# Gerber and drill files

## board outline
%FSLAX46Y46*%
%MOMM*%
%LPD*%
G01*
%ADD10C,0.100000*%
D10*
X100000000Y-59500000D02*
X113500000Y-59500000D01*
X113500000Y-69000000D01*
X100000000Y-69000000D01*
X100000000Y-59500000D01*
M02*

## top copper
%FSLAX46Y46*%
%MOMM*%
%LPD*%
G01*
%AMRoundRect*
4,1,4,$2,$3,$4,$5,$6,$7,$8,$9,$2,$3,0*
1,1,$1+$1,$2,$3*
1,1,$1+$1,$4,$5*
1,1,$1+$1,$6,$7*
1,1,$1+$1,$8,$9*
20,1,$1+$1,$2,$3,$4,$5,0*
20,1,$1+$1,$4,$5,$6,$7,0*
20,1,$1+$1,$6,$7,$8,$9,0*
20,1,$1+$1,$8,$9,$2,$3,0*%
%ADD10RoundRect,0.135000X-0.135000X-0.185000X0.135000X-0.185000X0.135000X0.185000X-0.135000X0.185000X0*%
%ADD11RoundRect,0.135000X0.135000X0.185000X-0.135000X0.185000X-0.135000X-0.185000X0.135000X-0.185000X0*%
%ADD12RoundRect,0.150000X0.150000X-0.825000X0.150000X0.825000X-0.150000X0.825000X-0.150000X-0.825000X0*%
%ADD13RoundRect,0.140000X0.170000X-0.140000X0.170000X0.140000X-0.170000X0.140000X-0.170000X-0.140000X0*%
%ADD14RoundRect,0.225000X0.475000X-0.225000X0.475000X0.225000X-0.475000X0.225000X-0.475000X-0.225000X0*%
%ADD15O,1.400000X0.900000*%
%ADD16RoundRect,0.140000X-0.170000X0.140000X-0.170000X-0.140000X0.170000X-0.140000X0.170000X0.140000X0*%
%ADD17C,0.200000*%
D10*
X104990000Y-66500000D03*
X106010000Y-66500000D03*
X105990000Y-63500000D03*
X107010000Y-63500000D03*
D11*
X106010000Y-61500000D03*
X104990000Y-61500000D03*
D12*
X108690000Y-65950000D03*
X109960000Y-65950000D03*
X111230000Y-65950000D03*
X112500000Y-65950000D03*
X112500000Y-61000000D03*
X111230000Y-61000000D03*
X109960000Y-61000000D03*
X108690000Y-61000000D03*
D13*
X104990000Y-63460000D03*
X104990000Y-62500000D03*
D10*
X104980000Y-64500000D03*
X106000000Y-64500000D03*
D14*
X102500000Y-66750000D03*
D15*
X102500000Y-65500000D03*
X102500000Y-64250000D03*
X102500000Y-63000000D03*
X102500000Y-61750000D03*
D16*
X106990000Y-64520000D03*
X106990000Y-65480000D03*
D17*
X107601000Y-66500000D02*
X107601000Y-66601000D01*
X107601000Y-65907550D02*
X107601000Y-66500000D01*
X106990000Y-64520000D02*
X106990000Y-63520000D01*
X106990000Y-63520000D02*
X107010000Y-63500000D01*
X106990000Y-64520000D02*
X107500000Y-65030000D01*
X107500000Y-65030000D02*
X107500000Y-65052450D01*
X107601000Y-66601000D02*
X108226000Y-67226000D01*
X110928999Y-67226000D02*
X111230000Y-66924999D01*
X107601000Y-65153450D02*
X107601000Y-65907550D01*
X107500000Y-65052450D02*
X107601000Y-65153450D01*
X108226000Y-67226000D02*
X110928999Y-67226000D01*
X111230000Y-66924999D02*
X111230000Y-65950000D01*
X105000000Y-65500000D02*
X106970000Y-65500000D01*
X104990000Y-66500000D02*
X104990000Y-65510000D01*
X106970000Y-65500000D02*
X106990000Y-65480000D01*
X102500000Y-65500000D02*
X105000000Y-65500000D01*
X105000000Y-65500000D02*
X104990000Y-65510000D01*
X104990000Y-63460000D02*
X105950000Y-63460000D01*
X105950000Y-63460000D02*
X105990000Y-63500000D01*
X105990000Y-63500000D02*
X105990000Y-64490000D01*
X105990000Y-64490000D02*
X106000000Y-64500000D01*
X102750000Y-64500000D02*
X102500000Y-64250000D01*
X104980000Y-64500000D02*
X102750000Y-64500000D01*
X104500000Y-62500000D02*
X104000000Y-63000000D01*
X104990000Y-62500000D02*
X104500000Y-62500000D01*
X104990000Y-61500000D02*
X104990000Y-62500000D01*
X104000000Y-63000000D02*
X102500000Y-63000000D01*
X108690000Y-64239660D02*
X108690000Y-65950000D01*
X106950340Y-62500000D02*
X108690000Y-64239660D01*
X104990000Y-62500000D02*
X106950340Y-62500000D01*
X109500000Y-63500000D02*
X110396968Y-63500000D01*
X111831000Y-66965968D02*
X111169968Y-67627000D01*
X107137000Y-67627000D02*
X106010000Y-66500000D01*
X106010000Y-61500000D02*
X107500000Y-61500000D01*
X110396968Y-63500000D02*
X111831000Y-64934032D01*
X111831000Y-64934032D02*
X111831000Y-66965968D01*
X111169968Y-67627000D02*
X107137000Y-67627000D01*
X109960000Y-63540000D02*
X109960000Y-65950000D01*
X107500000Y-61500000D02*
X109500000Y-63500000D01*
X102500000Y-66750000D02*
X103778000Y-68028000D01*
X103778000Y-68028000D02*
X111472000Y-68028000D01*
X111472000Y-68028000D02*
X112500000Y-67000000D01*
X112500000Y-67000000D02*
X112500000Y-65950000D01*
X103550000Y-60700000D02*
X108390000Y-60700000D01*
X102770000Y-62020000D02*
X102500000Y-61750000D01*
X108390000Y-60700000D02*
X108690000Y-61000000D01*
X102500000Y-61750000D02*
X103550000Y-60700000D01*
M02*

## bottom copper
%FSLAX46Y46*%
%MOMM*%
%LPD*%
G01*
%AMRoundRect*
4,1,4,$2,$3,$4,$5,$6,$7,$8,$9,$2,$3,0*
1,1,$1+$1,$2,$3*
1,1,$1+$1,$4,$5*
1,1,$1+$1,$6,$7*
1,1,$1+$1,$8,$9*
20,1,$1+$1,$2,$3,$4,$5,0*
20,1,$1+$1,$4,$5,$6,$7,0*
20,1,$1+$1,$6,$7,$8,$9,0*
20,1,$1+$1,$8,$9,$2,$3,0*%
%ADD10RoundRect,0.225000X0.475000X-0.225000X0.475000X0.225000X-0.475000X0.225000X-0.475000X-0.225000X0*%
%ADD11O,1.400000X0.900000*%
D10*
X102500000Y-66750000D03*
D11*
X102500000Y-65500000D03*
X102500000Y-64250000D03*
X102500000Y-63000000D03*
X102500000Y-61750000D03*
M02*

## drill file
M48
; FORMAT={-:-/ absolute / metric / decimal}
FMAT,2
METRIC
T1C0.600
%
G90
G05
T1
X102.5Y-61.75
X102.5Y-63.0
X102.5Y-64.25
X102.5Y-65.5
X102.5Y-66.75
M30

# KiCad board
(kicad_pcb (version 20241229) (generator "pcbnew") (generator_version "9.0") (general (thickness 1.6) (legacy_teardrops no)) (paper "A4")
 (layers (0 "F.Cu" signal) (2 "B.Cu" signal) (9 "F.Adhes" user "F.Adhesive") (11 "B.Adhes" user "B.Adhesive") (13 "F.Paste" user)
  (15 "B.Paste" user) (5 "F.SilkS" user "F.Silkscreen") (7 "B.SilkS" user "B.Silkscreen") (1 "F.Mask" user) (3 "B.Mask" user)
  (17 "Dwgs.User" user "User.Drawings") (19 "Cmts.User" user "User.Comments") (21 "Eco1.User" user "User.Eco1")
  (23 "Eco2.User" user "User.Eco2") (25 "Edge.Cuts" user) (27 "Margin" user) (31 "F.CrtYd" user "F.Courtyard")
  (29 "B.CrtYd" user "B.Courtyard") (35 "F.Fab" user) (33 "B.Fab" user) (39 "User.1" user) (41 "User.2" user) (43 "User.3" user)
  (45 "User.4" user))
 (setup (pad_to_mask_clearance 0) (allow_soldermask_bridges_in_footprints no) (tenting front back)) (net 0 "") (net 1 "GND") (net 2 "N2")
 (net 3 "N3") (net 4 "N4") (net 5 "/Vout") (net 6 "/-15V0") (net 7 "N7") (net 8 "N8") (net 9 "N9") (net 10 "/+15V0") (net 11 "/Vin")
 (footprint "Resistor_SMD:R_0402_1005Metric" (layer "F.Cu") (at 105.5 66.5)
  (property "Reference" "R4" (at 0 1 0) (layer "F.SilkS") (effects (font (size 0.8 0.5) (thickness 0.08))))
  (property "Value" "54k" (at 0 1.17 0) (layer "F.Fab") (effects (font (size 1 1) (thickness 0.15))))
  (pad "1" smd roundrect (at -0.51 0) (size 0.54 0.64) (layers "F.Cu" "F.Mask" "F.Paste") (roundrect_rratio 0.25) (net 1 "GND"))
  (pad "2" smd roundrect (at 0.51 0) (size 0.54 0.64) (layers "F.Cu" "F.Mask" "F.Paste") (roundrect_rratio 0.25) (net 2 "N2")))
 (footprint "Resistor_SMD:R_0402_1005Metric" (layer "F.Cu") (at 106.5 63.5)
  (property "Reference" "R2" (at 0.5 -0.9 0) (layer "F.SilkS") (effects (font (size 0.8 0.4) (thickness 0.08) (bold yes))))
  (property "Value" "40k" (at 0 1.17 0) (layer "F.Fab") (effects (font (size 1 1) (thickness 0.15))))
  (pad "1" smd roundrect (at -0.51 0) (size 0.54 0.64) (layers "F.Cu" "F.Mask" "F.Paste") (roundrect_rratio 0.25) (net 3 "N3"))
  (pad "2" smd roundrect (at 0.51 0) (size 0.54 0.64) (layers "F.Cu" "F.Mask" "F.Paste") (roundrect_rratio 0.25) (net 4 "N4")))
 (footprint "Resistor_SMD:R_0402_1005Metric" (layer "F.Cu") (at 105.5 61.5 180)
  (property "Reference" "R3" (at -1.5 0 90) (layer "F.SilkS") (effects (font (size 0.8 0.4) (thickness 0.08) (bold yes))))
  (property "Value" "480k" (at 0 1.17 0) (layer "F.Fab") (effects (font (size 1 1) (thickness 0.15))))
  (pad "1" smd roundrect (at -0.51 0 180) (size 0.54 0.64) (layers "F.Cu" "F.Mask" "F.Paste") (roundrect_rratio 0.25) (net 2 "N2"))
  (pad "2" smd roundrect (at 0.51 0 180) (size 0.54 0.64) (layers "F.Cu" "F.Mask" "F.Paste") (roundrect_rratio 0.25) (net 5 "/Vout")))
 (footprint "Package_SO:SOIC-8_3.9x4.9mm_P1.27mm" (layer "F.Cu") (at 110.595 63.475 90)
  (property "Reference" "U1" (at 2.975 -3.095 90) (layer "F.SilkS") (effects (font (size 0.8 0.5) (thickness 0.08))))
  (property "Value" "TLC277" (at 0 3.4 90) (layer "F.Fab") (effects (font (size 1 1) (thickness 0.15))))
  (pad "1" smd roundrect (at -2.475 -1.905 90) (size 1.95 0.6) (layers "F.Cu" "F.Mask" "F.Paste") (roundrect_rratio 0.25) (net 5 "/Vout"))
  (pad "2" smd roundrect (at -2.475 -0.635 90) (size 1.95 0.6) (layers "F.Cu" "F.Mask" "F.Paste") (roundrect_rratio 0.25) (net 2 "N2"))
  (pad "3" smd roundrect (at -2.475 0.635 90) (size 1.95 0.6) (layers "F.Cu" "F.Mask" "F.Paste") (roundrect_rratio 0.25) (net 4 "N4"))
  (pad "4" smd roundrect (at -2.475 1.905 90) (size 1.95 0.6) (layers "F.Cu" "F.Mask" "F.Paste") (roundrect_rratio 0.25) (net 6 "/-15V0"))
  (pad "5" smd roundrect (at 2.475 1.905 90) (size 1.95 0.6) (layers "F.Cu" "F.Mask" "F.Paste") (roundrect_rratio 0.25) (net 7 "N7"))
  (pad "6" smd roundrect (at 2.475 0.635 90) (size 1.95 0.6) (layers "F.Cu" "F.Mask" "F.Paste") (roundrect_rratio 0.25) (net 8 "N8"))
  (pad "7" smd roundrect (at 2.475 -0.635 90) (size 1.95 0.6) (layers "F.Cu" "F.Mask" "F.Paste") (roundrect_rratio 0.25) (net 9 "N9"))
  (pad "8" smd roundrect (at 2.475 -1.905 90) (size 1.95 0.6) (layers "F.Cu" "F.Mask" "F.Paste") (roundrect_rratio 0.25) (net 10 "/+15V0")))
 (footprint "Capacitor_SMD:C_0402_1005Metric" (layer "F.Cu") (at 104.99 62.98 90)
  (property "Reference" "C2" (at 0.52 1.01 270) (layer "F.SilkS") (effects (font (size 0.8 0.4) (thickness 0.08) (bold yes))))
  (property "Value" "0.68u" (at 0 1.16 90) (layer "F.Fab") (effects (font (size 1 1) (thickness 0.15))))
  (pad "1" smd roundrect (at -0.48 0 90) (size 0.56 0.62) (layers "F.Cu" "F.Mask" "F.Paste") (roundrect_rratio 0.25) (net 3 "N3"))
  (pad "2" smd roundrect (at 0.48 0 90) (size 0.56 0.62) (layers "F.Cu" "F.Mask" "F.Paste") (roundrect_rratio 0.25) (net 5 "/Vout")))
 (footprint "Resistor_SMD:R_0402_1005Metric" (layer "F.Cu") (at 105.49 64.5)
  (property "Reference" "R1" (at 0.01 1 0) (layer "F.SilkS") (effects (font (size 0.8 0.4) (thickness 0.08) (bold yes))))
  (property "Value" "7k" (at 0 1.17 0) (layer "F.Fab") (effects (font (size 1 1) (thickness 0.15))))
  (pad "1" smd roundrect (at -0.51 0) (size 0.54 0.64) (layers "F.Cu" "F.Mask" "F.Paste") (roundrect_rratio 0.25) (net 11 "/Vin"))
  (pad "2" smd roundrect (at 0.51 0) (size 0.54 0.64) (layers "F.Cu" "F.Mask" "F.Paste") (roundrect_rratio 0.25) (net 3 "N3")))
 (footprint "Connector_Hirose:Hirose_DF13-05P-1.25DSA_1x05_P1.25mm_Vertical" (layer "F.Cu") (at 102.5 66.75 90)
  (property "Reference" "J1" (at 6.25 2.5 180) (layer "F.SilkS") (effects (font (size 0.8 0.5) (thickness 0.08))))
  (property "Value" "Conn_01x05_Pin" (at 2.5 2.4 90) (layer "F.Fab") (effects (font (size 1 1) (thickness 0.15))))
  (pad "1" thru_hole roundrect (at 0 0 90) (size 0.9 1.4) (drill 0.6) (layers "*.Cu" "*.Mask") (remove_unused_layers no)
   (roundrect_rratio 0.25) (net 6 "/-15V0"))
  (pad "2" thru_hole oval (at 1.25 0 90) (size 0.9 1.4) (drill 0.6) (layers "*.Cu" "*.Mask") (remove_unused_layers no) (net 1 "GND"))
  (pad "3" thru_hole oval (at 2.5 0 90) (size 0.9 1.4) (drill 0.6) (layers "*.Cu" "*.Mask") (remove_unused_layers no) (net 11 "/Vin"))
  (pad "4" thru_hole oval (at 3.75 0 90) (size 0.9 1.4) (drill 0.6) (layers "*.Cu" "*.Mask") (remove_unused_layers no) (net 5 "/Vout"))
  (pad "5" thru_hole oval (at 5 0 90) (size 0.9 1.4) (drill 0.6) (layers "*.Cu" "*.Mask") (remove_unused_layers no) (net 10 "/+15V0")))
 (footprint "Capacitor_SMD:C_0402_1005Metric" (layer "F.Cu") (at 106.99 65 -90)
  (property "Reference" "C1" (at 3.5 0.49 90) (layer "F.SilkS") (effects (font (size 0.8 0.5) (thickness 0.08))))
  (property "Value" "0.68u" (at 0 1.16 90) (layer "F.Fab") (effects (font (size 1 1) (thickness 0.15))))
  (pad "1" smd roundrect (at -0.48 0 270) (size 0.56 0.62) (layers "F.Cu" "F.Mask" "F.Paste") (roundrect_rratio 0.25) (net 4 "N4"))
  (pad "2" smd roundrect (at 0.48 0 270) (size 0.56 0.62) (layers "F.Cu" "F.Mask" "F.Paste") (roundrect_rratio 0.25) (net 1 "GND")))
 (gr_rect (start 100 59.5) (end 113.5 69) (stroke (width 0.1) (type solid)) (fill no) (layer "Edge.Cuts"))
 (segment (start 107.601 66.5) (end 107.601 66.601) (width 0.2) (layer "F.Cu") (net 4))
 (segment (start 107.601 65.90755) (end 107.601 66.5) (width 0.2) (layer "F.Cu") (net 4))
 (segment (start 106.99 64.52) (end 106.99 63.52) (width 0.2) (layer "F.Cu") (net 4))
 (segment (start 106.99 63.52) (end 107.01 63.5) (width 0.2) (layer "F.Cu") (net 4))
 (segment (start 106.99 64.52) (end 107.5 65.03) (width 0.2) (layer "F.Cu") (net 4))
 (segment (start 107.5 65.03) (end 107.5 65.05245) (width 0.2) (layer "F.Cu") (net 4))
 (segment (start 107.601 66.601) (end 108.226 67.226) (width 0.2) (layer "F.Cu") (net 4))
 (segment (start 110.928999 67.226) (end 111.23 66.924999) (width 0.2) (layer "F.Cu") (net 4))
 (segment (start 107.601 65.15345) (end 107.601 65.90755) (width 0.2) (layer "F.Cu") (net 4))
 (segment (start 107.5 65.05245) (end 107.601 65.15345) (width 0.2) (layer "F.Cu") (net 4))
 (segment (start 108.226 67.226) (end 110.928999 67.226) (width 0.2) (layer "F.Cu") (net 4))
 (segment (start 111.23 66.924999) (end 111.23 65.95) (width 0.2) (layer "F.Cu") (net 4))
 (segment (start 105 65.5) (end 106.97 65.5) (width 0.2) (layer "F.Cu") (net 1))
 (segment (start 104.99 66.5) (end 104.99 65.51) (width 0.2) (layer "F.Cu") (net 1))
 (segment (start 106.97 65.5) (end 106.99 65.48) (width 0.2) (layer "F.Cu") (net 1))
 (segment (start 102.5 65.5) (end 105 65.5) (width 0.2) (layer "F.Cu") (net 1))
 (segment (start 105 65.5) (end 104.99 65.51) (width 0.2) (layer "F.Cu") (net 1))
 (segment (start 104.99 63.46) (end 105.95 63.46) (width 0.2) (layer "F.Cu") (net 3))
 (segment (start 105.95 63.46) (end 105.99 63.5) (width 0.2) (layer "F.Cu") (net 3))
 (segment (start 105.99 63.5) (end 105.99 64.49) (width 0.2) (layer "F.Cu") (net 3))
 (segment (start 105.99 64.49) (end 106 64.5) (width 0.2) (layer "F.Cu") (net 3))
 (segment (start 102.75 64.5) (end 102.5 64.25) (width 0.2) (layer "F.Cu") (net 11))
 (segment (start 104.98 64.5) (end 102.75 64.5) (width 0.2) (layer "F.Cu") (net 11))
 (segment (start 104.5 62.5) (end 104 63) (width 0.2) (layer "F.Cu") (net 5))
 (segment (start 104.99 62.5) (end 104.5 62.5) (width 0.2) (layer "F.Cu") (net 5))
 (segment (start 104.99 61.5) (end 104.99 62.5) (width 0.2) (layer "F.Cu") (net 5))
 (segment (start 104 63) (end 102.5 63) (width 0.2) (layer "F.Cu") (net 5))
 (segment (start 108.69 64.23966) (end 108.69 65.95) (width 0.2) (layer "F.Cu") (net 5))
 (segment (start 106.95034 62.5) (end 108.69 64.23966) (width 0.2) (layer "F.Cu") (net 5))
 (segment (start 104.99 62.5) (end 106.95034 62.5) (width 0.2) (layer "F.Cu") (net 5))
 (segment (start 109.5 63.5) (end 110.396968 63.5) (width 0.2) (layer "F.Cu") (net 2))
 (segment (start 111.831 66.965968) (end 111.169968 67.627) (width 0.2) (layer "F.Cu") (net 2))
 (segment (start 107.137 67.627) (end 106.01 66.5) (width 0.2) (layer "F.Cu") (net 2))
 (segment (start 106.01 61.5) (end 107.5 61.5) (width 0.2) (layer "F.Cu") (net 2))
 (segment (start 110.396968 63.5) (end 111.831 64.934032) (width 0.2) (layer "F.Cu") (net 2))
 (segment (start 111.831 64.934032) (end 111.831 66.965968) (width 0.2) (layer "F.Cu") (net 2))
 (segment (start 111.169968 67.627) (end 107.137 67.627) (width 0.2) (layer "F.Cu") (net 2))
 (segment (start 109.96 63.54) (end 109.96 65.95) (width 0.2) (layer "F.Cu") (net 2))
 (segment (start 107.5 61.5) (end 109.5 63.5) (width 0.2) (layer "F.Cu") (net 2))
 (segment (start 102.5 66.75) (end 103.778 68.028) (width 0.2) (layer "F.Cu") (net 6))
 (segment (start 103.778 68.028) (end 111.472 68.028) (width 0.2) (layer "F.Cu") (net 6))
 (segment (start 111.472 68.028) (end 112.5 67) (width 0.2) (layer "F.Cu") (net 6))
 (segment (start 112.5 67) (end 112.5 65.95) (width 0.2) (layer "F.Cu") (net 6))
 (segment (start 103.55 60.7) (end 108.39 60.7) (width 0.2) (layer "F.Cu") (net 10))
 (segment (start 102.77 62.02) (end 102.5 61.75) (width 0.2) (layer "F.Cu") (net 10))
 (segment (start 108.39 60.7) (end 108.69 61) (width 0.2) (layer "F.Cu") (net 10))
 (segment (start 102.5 61.75) (end 103.55 60.7) (width 0.2) (layer "F.Cu") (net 10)))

